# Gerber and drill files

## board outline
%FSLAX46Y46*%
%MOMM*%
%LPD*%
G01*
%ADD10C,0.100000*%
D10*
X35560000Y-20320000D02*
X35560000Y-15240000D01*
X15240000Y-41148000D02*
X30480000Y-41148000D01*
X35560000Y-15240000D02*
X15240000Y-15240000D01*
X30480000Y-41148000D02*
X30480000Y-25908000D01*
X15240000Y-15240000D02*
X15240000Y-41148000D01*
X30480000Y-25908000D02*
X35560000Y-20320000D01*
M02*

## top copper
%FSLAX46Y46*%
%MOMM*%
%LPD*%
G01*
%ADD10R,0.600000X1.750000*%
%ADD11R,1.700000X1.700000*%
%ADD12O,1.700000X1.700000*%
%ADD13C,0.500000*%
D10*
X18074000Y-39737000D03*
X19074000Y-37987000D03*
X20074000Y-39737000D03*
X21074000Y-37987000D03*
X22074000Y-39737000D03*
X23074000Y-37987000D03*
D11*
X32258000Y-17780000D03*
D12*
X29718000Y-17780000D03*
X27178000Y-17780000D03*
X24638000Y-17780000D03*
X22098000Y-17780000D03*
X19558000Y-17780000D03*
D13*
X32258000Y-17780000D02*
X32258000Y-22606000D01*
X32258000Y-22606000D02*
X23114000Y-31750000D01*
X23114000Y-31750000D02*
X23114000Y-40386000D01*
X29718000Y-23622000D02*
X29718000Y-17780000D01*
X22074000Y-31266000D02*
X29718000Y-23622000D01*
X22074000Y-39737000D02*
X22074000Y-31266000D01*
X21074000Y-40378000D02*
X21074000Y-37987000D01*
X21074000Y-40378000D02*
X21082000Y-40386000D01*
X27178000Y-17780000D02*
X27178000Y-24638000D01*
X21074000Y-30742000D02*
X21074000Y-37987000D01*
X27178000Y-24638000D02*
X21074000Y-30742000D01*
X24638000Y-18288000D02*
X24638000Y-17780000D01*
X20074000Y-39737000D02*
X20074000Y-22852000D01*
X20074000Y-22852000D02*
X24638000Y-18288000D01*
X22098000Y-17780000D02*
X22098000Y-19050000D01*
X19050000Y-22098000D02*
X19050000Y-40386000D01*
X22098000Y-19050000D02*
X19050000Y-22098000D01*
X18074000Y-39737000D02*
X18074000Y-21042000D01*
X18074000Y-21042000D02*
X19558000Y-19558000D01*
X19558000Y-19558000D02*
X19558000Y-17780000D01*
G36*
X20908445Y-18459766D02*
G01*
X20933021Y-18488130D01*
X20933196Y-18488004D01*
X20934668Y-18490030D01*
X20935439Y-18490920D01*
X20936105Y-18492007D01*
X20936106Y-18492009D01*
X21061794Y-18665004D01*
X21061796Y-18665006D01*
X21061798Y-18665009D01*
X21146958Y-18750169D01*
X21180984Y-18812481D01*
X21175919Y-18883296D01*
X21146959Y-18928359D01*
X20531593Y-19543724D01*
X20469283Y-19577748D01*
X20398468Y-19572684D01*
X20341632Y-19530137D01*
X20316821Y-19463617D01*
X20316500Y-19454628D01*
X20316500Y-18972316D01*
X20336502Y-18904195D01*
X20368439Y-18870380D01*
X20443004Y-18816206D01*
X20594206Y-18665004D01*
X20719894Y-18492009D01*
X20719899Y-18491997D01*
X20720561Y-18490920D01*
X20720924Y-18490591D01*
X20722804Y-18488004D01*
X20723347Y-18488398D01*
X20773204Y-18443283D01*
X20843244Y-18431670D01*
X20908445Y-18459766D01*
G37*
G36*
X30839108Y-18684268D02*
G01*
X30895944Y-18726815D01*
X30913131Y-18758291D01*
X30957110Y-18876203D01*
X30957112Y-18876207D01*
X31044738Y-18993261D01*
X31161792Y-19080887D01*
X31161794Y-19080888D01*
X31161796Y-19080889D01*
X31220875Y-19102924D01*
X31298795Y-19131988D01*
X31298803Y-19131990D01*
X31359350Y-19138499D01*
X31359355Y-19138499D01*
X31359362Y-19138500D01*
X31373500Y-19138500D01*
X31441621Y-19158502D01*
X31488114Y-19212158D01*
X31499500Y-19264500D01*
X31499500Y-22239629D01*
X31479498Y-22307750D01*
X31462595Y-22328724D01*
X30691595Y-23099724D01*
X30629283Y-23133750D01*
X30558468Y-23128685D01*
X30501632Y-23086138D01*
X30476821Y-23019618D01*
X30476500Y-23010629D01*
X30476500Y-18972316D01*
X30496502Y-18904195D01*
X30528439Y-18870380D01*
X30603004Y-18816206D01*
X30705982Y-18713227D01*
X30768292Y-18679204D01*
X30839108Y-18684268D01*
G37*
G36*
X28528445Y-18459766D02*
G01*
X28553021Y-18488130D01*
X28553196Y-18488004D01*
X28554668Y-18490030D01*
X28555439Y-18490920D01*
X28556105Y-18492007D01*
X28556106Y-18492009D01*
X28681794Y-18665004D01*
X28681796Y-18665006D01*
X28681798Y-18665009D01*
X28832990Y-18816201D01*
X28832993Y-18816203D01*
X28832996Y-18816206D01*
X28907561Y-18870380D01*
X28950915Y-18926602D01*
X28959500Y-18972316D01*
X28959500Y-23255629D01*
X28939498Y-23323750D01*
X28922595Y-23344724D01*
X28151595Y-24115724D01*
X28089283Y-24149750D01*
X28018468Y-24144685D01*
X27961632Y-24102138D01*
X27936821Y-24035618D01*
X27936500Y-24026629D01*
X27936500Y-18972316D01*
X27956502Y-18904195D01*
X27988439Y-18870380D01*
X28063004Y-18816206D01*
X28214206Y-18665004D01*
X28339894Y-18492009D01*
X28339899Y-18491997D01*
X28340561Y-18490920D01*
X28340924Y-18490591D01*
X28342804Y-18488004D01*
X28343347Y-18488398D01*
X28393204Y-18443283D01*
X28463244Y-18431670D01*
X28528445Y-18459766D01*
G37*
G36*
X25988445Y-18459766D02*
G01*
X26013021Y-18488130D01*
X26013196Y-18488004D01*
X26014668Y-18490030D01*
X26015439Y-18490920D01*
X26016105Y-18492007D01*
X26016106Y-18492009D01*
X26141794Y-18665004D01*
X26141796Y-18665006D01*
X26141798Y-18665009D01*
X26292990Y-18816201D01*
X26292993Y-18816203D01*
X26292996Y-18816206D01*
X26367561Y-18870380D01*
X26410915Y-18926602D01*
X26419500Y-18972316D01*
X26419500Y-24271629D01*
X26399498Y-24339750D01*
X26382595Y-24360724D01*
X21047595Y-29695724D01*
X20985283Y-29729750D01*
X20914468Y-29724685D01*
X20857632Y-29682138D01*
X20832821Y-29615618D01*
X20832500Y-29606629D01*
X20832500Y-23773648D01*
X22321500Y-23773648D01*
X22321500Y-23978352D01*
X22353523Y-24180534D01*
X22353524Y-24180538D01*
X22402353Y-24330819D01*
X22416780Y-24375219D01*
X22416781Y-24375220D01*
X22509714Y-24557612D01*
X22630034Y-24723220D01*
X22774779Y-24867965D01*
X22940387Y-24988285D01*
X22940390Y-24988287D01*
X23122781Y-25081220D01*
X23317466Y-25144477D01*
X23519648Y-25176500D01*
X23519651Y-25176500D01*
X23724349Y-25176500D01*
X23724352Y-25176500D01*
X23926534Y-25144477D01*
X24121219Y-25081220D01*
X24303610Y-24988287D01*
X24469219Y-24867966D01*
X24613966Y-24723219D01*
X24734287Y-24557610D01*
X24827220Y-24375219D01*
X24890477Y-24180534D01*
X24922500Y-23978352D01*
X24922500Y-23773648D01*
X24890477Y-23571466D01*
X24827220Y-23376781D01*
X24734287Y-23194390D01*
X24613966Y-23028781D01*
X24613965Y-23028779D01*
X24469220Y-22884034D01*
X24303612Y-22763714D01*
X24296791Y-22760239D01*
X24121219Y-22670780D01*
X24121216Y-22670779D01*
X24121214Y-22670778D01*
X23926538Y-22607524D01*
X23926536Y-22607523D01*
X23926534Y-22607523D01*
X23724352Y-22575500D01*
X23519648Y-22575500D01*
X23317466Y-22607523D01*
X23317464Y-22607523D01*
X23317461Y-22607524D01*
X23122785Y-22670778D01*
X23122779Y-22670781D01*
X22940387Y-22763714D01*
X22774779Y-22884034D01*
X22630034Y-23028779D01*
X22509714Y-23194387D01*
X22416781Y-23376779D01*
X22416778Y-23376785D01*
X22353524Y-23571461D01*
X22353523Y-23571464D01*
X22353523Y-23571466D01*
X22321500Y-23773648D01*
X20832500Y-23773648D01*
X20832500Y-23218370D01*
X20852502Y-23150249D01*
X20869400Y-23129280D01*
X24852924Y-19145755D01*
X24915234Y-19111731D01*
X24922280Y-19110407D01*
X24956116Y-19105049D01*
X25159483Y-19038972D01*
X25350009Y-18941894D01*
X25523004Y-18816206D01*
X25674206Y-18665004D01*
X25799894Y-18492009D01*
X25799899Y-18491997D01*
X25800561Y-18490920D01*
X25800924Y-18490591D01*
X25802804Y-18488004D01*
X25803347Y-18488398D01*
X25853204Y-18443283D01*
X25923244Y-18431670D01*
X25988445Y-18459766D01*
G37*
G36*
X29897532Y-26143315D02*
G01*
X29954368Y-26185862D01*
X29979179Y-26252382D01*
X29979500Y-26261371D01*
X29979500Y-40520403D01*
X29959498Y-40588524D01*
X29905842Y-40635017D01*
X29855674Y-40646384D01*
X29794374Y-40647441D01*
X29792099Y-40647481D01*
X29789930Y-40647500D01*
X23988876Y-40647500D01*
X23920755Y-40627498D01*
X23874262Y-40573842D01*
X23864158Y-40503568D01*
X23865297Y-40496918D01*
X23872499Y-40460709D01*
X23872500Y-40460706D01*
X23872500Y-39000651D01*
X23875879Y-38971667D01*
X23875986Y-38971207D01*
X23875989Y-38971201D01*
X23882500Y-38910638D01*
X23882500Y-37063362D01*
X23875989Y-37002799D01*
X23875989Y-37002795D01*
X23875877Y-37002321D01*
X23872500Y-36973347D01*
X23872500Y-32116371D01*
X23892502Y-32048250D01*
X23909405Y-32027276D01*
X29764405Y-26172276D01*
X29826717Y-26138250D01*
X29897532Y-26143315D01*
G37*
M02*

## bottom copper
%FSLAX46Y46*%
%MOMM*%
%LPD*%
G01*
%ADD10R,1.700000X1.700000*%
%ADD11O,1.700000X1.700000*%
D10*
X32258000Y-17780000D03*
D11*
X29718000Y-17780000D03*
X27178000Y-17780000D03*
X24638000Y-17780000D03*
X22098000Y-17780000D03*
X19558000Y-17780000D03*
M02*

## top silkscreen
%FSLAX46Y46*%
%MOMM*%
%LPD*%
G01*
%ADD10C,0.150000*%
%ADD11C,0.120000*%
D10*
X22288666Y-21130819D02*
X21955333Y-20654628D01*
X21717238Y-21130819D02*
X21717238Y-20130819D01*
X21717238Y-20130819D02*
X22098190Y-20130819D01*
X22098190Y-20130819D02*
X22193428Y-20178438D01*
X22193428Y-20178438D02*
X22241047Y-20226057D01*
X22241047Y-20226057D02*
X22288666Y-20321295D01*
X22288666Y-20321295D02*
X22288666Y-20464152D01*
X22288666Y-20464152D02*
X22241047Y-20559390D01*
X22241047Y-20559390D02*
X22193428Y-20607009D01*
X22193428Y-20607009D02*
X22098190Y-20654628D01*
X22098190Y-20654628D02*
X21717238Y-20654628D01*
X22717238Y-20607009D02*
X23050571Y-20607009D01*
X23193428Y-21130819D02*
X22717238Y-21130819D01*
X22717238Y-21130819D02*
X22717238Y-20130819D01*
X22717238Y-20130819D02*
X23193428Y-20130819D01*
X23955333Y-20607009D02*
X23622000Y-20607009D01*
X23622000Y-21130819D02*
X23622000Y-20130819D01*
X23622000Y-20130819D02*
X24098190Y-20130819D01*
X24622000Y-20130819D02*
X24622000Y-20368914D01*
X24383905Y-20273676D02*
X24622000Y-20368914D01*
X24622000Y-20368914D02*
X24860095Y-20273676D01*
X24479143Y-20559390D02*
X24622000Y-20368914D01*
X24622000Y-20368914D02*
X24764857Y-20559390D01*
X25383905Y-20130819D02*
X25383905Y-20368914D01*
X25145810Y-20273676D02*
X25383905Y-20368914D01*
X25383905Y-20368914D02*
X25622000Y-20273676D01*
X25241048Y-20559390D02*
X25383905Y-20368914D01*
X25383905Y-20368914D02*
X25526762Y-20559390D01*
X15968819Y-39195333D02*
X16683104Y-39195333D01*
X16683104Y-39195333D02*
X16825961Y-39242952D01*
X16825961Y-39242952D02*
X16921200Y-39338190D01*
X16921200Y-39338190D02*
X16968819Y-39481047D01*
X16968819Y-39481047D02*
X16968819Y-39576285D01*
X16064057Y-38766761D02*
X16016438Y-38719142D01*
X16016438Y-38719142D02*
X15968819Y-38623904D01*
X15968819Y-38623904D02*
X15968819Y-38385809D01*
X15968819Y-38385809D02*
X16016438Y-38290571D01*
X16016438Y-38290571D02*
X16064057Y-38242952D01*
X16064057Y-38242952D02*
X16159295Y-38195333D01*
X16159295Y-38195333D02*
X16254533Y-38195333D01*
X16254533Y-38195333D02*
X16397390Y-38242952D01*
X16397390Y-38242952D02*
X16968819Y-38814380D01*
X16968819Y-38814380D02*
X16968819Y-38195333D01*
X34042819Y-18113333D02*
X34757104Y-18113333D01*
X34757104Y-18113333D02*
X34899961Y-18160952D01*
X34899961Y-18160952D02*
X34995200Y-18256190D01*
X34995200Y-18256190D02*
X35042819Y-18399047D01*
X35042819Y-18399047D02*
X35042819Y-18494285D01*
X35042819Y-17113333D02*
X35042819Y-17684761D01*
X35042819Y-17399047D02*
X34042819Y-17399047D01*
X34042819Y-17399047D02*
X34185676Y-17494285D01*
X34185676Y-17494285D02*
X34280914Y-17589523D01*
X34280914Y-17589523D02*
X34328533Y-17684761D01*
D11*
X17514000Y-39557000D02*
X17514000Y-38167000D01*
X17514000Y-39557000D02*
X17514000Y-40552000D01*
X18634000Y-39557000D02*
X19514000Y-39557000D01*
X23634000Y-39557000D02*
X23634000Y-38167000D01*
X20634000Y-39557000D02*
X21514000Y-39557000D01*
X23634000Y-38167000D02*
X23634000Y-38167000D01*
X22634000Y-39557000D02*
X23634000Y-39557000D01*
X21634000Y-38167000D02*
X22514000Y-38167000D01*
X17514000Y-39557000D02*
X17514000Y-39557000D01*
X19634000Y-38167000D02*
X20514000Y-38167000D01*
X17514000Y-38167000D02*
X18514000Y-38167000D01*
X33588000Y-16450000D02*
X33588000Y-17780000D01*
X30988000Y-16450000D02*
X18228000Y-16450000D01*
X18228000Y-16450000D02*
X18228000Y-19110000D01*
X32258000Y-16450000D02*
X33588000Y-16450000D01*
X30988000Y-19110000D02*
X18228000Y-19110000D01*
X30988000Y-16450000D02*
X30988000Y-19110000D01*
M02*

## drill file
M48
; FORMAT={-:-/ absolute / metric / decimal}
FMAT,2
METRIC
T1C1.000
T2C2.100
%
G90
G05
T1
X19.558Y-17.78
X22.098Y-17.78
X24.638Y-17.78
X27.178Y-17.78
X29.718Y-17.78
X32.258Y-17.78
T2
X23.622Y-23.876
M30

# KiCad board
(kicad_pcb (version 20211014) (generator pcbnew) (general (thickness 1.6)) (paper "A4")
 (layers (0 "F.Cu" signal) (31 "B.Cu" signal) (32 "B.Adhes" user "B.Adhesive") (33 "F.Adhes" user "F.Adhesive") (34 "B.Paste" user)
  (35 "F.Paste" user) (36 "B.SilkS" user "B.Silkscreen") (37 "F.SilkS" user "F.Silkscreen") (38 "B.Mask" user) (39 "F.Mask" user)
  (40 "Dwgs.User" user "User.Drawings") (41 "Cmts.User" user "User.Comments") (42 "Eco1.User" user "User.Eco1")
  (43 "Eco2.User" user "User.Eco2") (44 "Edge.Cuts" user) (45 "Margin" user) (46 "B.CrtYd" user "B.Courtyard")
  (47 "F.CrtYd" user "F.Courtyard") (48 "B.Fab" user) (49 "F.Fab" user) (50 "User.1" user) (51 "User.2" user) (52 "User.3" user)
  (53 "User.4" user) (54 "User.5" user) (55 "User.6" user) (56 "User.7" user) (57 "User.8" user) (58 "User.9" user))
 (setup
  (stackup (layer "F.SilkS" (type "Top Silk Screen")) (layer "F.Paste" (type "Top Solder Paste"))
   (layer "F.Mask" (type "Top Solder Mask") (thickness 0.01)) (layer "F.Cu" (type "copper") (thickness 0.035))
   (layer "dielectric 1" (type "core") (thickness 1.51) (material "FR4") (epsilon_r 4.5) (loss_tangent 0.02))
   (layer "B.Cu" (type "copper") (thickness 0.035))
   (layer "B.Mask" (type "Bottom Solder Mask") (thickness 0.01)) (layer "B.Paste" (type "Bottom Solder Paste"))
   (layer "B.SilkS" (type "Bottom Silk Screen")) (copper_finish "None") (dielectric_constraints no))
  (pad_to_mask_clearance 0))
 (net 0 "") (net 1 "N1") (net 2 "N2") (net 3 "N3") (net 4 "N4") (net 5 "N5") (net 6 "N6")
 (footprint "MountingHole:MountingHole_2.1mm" (layer "F.Cu") (at 23.622 23.876)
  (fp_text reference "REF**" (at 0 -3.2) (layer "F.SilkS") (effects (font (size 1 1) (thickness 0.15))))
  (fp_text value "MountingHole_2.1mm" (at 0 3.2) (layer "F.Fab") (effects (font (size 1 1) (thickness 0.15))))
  (pad "" np_thru_hole circle (at 0 0) (size 2.1 2.1) (drill 2.1) (layers *.Cu *.Mask)))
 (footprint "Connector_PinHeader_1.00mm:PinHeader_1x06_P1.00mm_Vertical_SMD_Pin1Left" (layer "F.Cu") (at 20.574 38.862 90)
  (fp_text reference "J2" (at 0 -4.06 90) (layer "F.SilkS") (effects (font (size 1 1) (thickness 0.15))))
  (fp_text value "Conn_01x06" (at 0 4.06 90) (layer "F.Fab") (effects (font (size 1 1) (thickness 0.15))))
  (fp_line (start -0.695 -3.06) (end 0.695 -3.06) (layer "F.SilkS") (width 0.12))
  (fp_line (start -0.695 -3.06) (end -1.69 -3.06) (layer "F.SilkS") (width 0.12))
  (fp_line (start -0.695 -1.94) (end -0.695 -1.06) (layer "F.SilkS") (width 0.12))
  (fp_line (start -0.695 3.06) (end 0.695 3.06) (layer "F.SilkS") (width 0.12))
  (fp_line (start -0.695 0.06) (end -0.695 0.94) (layer "F.SilkS") (width 0.12))
  (fp_line (start 0.695 3.06) (end 0.695 3.06) (layer "F.SilkS") (width 0.12))
  (fp_line (start -0.695 2.06) (end -0.695 3.06) (layer "F.SilkS") (width 0.12))
  (fp_line (start 0.695 1.06) (end 0.695 1.94) (layer "F.SilkS") (width 0.12))
  (fp_line (start -0.695 -3.06) (end -0.695 -3.06) (layer "F.SilkS") (width 0.12))
  (fp_line (start 0.695 -0.94) (end 0.695 -0.06) (layer "F.SilkS") (width 0.12))
  (fp_line (start 0.695 -3.06) (end 0.695 -2.06) (layer "F.SilkS") (width 0.12))
  (pad "1" smd rect (at -0.875 -2.5 90) (size 1.75 0.6) (layers "F.Cu" "F.Paste" "F.Mask") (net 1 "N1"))
  (pad "2" smd rect (at 0.875 -1.5 90) (size 1.75 0.6) (layers "F.Cu" "F.Paste" "F.Mask") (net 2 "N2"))
  (pad "3" smd rect (at -0.875 -0.5 90) (size 1.75 0.6) (layers "F.Cu" "F.Paste" "F.Mask") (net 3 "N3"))
  (pad "4" smd rect (at 0.875 0.5 90) (size 1.75 0.6) (layers "F.Cu" "F.Paste" "F.Mask") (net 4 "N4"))
  (pad "5" smd rect (at -0.875 1.5 90) (size 1.75 0.6) (layers "F.Cu" "F.Paste" "F.Mask") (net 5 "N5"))
  (pad "6" smd rect (at 0.875 2.5 90) (size 1.75 0.6) (layers "F.Cu" "F.Paste" "F.Mask") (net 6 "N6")))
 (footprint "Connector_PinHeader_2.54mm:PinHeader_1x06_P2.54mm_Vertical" (layer "F.Cu") (at 32.258 17.78 -90)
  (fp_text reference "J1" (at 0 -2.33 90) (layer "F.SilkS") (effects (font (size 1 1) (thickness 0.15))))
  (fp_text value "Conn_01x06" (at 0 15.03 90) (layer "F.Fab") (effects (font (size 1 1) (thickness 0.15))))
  (fp_line (start -1.33 -1.33) (end 0 -1.33) (layer "F.SilkS") (width 0.12))
  (fp_line (start -1.33 1.27) (end -1.33 14.03) (layer "F.SilkS") (width 0.12))
  (fp_line (start -1.33 14.03) (end 1.33 14.03) (layer "F.SilkS") (width 0.12))
  (fp_line (start -1.33 0) (end -1.33 -1.33) (layer "F.SilkS") (width 0.12))
  (fp_line (start 1.33 1.27) (end 1.33 14.03) (layer "F.SilkS") (width 0.12))
  (fp_line (start -1.33 1.27) (end 1.33 1.27) (layer "F.SilkS") (width 0.12))
  (pad "1" thru_hole rect (at 0 0 270) (size 1.7 1.7) (drill 1) (layers *.Cu *.Mask) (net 6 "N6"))
  (pad "2" thru_hole oval (at 0 2.54 270) (size 1.7 1.7) (drill 1) (layers *.Cu *.Mask) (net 5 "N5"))
  (pad "3" thru_hole oval (at 0 5.08 270) (size 1.7 1.7) (drill 1) (layers *.Cu *.Mask) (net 4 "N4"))
  (pad "4" thru_hole oval (at 0 7.62 270) (size 1.7 1.7) (drill 1) (layers *.Cu *.Mask) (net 3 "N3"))
  (pad "5" thru_hole oval (at 0 10.16 270) (size 1.7 1.7) (drill 1) (layers *.Cu *.Mask) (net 2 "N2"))
  (pad "6" thru_hole oval (at 0 12.7 270) (size 1.7 1.7) (drill 1) (layers *.Cu *.Mask) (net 1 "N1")))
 (gr_line (start 35.56 20.32) (end 35.56 15.24) (layer "Edge.Cuts") (width 0.1))
 (gr_line (start 15.24 41.148) (end 30.48 41.148) (layer "Edge.Cuts") (width 0.1))
 (gr_line (start 35.56 15.24) (end 15.24 15.24) (layer "Edge.Cuts") (width 0.1))
 (gr_line (start 30.48 41.148) (end 30.48 25.908) (layer "Edge.Cuts") (width 0.1))
 (gr_line (start 15.24 15.24) (end 15.24 41.148) (layer "Edge.Cuts") (width 0.1))
 (gr_line (start 30.48 25.908) (end 35.56 20.32) (layer "Edge.Cuts") (width 0.1))
 (segment (start 32.258 17.78) (end 32.258 22.606) (width 0.5) (layer "F.Cu") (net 6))
 (segment (start 32.258 22.606) (end 23.114 31.75) (width 0.5) (layer "F.Cu") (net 6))
 (segment (start 23.114 31.75) (end 23.114 40.386) (width 0.5) (layer "F.Cu") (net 6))
 (segment (start 29.718 23.622) (end 29.718 17.78) (width 0.5) (layer "F.Cu") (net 5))
 (segment (start 22.074 31.266) (end 29.718 23.622) (width 0.5) (layer "F.Cu") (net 5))
 (segment (start 22.074 39.737) (end 22.074 31.266) (width 0.5) (layer "F.Cu") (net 5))
 (segment (start 21.074 40.378) (end 21.074 37.987) (width 0.5) (layer "F.Cu") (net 4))
 (segment (start 21.074 40.378) (end 21.082 40.386) (width 0.5) (layer "F.Cu") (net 4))
 (segment (start 27.178 17.78) (end 27.178 24.638) (width 0.5) (layer "F.Cu") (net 4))
 (segment (start 21.074 30.742) (end 21.074 37.987) (width 0.5) (layer "F.Cu") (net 4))
 (segment (start 27.178 24.638) (end 21.074 30.742) (width 0.5) (layer "F.Cu") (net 4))
 (segment (start 24.638 18.288) (end 24.638 17.78) (width 0.5) (layer "F.Cu") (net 3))
 (segment (start 20.074 39.737) (end 20.074 22.852) (width 0.5) (layer "F.Cu") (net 3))
 (segment (start 20.074 22.852) (end 24.638 18.288) (width 0.5) (layer "F.Cu") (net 3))
 (segment (start 22.098 17.78) (end 22.098 19.05) (width 0.5) (layer "F.Cu") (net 2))
 (segment (start 19.05 22.098) (end 19.05 40.386) (width 0.5) (layer "F.Cu") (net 2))
 (segment (start 22.098 19.05) (end 19.05 22.098) (width 0.5) (layer "F.Cu") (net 2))
 (segment (start 18.074 39.737) (end 18.074 21.042) (width 0.5) (layer "F.Cu") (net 1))
 (segment (start 18.074 21.042) (end 19.558 19.558) (width 0.5) (layer "F.Cu") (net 1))
 (segment (start 19.558 19.558) (end 19.558 17.78) (width 0.5) (layer "F.Cu") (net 1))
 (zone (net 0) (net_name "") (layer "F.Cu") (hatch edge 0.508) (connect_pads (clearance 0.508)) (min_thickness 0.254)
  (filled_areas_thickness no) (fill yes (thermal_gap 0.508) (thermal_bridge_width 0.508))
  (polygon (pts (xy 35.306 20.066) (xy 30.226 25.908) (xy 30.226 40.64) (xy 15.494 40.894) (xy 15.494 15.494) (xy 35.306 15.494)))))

